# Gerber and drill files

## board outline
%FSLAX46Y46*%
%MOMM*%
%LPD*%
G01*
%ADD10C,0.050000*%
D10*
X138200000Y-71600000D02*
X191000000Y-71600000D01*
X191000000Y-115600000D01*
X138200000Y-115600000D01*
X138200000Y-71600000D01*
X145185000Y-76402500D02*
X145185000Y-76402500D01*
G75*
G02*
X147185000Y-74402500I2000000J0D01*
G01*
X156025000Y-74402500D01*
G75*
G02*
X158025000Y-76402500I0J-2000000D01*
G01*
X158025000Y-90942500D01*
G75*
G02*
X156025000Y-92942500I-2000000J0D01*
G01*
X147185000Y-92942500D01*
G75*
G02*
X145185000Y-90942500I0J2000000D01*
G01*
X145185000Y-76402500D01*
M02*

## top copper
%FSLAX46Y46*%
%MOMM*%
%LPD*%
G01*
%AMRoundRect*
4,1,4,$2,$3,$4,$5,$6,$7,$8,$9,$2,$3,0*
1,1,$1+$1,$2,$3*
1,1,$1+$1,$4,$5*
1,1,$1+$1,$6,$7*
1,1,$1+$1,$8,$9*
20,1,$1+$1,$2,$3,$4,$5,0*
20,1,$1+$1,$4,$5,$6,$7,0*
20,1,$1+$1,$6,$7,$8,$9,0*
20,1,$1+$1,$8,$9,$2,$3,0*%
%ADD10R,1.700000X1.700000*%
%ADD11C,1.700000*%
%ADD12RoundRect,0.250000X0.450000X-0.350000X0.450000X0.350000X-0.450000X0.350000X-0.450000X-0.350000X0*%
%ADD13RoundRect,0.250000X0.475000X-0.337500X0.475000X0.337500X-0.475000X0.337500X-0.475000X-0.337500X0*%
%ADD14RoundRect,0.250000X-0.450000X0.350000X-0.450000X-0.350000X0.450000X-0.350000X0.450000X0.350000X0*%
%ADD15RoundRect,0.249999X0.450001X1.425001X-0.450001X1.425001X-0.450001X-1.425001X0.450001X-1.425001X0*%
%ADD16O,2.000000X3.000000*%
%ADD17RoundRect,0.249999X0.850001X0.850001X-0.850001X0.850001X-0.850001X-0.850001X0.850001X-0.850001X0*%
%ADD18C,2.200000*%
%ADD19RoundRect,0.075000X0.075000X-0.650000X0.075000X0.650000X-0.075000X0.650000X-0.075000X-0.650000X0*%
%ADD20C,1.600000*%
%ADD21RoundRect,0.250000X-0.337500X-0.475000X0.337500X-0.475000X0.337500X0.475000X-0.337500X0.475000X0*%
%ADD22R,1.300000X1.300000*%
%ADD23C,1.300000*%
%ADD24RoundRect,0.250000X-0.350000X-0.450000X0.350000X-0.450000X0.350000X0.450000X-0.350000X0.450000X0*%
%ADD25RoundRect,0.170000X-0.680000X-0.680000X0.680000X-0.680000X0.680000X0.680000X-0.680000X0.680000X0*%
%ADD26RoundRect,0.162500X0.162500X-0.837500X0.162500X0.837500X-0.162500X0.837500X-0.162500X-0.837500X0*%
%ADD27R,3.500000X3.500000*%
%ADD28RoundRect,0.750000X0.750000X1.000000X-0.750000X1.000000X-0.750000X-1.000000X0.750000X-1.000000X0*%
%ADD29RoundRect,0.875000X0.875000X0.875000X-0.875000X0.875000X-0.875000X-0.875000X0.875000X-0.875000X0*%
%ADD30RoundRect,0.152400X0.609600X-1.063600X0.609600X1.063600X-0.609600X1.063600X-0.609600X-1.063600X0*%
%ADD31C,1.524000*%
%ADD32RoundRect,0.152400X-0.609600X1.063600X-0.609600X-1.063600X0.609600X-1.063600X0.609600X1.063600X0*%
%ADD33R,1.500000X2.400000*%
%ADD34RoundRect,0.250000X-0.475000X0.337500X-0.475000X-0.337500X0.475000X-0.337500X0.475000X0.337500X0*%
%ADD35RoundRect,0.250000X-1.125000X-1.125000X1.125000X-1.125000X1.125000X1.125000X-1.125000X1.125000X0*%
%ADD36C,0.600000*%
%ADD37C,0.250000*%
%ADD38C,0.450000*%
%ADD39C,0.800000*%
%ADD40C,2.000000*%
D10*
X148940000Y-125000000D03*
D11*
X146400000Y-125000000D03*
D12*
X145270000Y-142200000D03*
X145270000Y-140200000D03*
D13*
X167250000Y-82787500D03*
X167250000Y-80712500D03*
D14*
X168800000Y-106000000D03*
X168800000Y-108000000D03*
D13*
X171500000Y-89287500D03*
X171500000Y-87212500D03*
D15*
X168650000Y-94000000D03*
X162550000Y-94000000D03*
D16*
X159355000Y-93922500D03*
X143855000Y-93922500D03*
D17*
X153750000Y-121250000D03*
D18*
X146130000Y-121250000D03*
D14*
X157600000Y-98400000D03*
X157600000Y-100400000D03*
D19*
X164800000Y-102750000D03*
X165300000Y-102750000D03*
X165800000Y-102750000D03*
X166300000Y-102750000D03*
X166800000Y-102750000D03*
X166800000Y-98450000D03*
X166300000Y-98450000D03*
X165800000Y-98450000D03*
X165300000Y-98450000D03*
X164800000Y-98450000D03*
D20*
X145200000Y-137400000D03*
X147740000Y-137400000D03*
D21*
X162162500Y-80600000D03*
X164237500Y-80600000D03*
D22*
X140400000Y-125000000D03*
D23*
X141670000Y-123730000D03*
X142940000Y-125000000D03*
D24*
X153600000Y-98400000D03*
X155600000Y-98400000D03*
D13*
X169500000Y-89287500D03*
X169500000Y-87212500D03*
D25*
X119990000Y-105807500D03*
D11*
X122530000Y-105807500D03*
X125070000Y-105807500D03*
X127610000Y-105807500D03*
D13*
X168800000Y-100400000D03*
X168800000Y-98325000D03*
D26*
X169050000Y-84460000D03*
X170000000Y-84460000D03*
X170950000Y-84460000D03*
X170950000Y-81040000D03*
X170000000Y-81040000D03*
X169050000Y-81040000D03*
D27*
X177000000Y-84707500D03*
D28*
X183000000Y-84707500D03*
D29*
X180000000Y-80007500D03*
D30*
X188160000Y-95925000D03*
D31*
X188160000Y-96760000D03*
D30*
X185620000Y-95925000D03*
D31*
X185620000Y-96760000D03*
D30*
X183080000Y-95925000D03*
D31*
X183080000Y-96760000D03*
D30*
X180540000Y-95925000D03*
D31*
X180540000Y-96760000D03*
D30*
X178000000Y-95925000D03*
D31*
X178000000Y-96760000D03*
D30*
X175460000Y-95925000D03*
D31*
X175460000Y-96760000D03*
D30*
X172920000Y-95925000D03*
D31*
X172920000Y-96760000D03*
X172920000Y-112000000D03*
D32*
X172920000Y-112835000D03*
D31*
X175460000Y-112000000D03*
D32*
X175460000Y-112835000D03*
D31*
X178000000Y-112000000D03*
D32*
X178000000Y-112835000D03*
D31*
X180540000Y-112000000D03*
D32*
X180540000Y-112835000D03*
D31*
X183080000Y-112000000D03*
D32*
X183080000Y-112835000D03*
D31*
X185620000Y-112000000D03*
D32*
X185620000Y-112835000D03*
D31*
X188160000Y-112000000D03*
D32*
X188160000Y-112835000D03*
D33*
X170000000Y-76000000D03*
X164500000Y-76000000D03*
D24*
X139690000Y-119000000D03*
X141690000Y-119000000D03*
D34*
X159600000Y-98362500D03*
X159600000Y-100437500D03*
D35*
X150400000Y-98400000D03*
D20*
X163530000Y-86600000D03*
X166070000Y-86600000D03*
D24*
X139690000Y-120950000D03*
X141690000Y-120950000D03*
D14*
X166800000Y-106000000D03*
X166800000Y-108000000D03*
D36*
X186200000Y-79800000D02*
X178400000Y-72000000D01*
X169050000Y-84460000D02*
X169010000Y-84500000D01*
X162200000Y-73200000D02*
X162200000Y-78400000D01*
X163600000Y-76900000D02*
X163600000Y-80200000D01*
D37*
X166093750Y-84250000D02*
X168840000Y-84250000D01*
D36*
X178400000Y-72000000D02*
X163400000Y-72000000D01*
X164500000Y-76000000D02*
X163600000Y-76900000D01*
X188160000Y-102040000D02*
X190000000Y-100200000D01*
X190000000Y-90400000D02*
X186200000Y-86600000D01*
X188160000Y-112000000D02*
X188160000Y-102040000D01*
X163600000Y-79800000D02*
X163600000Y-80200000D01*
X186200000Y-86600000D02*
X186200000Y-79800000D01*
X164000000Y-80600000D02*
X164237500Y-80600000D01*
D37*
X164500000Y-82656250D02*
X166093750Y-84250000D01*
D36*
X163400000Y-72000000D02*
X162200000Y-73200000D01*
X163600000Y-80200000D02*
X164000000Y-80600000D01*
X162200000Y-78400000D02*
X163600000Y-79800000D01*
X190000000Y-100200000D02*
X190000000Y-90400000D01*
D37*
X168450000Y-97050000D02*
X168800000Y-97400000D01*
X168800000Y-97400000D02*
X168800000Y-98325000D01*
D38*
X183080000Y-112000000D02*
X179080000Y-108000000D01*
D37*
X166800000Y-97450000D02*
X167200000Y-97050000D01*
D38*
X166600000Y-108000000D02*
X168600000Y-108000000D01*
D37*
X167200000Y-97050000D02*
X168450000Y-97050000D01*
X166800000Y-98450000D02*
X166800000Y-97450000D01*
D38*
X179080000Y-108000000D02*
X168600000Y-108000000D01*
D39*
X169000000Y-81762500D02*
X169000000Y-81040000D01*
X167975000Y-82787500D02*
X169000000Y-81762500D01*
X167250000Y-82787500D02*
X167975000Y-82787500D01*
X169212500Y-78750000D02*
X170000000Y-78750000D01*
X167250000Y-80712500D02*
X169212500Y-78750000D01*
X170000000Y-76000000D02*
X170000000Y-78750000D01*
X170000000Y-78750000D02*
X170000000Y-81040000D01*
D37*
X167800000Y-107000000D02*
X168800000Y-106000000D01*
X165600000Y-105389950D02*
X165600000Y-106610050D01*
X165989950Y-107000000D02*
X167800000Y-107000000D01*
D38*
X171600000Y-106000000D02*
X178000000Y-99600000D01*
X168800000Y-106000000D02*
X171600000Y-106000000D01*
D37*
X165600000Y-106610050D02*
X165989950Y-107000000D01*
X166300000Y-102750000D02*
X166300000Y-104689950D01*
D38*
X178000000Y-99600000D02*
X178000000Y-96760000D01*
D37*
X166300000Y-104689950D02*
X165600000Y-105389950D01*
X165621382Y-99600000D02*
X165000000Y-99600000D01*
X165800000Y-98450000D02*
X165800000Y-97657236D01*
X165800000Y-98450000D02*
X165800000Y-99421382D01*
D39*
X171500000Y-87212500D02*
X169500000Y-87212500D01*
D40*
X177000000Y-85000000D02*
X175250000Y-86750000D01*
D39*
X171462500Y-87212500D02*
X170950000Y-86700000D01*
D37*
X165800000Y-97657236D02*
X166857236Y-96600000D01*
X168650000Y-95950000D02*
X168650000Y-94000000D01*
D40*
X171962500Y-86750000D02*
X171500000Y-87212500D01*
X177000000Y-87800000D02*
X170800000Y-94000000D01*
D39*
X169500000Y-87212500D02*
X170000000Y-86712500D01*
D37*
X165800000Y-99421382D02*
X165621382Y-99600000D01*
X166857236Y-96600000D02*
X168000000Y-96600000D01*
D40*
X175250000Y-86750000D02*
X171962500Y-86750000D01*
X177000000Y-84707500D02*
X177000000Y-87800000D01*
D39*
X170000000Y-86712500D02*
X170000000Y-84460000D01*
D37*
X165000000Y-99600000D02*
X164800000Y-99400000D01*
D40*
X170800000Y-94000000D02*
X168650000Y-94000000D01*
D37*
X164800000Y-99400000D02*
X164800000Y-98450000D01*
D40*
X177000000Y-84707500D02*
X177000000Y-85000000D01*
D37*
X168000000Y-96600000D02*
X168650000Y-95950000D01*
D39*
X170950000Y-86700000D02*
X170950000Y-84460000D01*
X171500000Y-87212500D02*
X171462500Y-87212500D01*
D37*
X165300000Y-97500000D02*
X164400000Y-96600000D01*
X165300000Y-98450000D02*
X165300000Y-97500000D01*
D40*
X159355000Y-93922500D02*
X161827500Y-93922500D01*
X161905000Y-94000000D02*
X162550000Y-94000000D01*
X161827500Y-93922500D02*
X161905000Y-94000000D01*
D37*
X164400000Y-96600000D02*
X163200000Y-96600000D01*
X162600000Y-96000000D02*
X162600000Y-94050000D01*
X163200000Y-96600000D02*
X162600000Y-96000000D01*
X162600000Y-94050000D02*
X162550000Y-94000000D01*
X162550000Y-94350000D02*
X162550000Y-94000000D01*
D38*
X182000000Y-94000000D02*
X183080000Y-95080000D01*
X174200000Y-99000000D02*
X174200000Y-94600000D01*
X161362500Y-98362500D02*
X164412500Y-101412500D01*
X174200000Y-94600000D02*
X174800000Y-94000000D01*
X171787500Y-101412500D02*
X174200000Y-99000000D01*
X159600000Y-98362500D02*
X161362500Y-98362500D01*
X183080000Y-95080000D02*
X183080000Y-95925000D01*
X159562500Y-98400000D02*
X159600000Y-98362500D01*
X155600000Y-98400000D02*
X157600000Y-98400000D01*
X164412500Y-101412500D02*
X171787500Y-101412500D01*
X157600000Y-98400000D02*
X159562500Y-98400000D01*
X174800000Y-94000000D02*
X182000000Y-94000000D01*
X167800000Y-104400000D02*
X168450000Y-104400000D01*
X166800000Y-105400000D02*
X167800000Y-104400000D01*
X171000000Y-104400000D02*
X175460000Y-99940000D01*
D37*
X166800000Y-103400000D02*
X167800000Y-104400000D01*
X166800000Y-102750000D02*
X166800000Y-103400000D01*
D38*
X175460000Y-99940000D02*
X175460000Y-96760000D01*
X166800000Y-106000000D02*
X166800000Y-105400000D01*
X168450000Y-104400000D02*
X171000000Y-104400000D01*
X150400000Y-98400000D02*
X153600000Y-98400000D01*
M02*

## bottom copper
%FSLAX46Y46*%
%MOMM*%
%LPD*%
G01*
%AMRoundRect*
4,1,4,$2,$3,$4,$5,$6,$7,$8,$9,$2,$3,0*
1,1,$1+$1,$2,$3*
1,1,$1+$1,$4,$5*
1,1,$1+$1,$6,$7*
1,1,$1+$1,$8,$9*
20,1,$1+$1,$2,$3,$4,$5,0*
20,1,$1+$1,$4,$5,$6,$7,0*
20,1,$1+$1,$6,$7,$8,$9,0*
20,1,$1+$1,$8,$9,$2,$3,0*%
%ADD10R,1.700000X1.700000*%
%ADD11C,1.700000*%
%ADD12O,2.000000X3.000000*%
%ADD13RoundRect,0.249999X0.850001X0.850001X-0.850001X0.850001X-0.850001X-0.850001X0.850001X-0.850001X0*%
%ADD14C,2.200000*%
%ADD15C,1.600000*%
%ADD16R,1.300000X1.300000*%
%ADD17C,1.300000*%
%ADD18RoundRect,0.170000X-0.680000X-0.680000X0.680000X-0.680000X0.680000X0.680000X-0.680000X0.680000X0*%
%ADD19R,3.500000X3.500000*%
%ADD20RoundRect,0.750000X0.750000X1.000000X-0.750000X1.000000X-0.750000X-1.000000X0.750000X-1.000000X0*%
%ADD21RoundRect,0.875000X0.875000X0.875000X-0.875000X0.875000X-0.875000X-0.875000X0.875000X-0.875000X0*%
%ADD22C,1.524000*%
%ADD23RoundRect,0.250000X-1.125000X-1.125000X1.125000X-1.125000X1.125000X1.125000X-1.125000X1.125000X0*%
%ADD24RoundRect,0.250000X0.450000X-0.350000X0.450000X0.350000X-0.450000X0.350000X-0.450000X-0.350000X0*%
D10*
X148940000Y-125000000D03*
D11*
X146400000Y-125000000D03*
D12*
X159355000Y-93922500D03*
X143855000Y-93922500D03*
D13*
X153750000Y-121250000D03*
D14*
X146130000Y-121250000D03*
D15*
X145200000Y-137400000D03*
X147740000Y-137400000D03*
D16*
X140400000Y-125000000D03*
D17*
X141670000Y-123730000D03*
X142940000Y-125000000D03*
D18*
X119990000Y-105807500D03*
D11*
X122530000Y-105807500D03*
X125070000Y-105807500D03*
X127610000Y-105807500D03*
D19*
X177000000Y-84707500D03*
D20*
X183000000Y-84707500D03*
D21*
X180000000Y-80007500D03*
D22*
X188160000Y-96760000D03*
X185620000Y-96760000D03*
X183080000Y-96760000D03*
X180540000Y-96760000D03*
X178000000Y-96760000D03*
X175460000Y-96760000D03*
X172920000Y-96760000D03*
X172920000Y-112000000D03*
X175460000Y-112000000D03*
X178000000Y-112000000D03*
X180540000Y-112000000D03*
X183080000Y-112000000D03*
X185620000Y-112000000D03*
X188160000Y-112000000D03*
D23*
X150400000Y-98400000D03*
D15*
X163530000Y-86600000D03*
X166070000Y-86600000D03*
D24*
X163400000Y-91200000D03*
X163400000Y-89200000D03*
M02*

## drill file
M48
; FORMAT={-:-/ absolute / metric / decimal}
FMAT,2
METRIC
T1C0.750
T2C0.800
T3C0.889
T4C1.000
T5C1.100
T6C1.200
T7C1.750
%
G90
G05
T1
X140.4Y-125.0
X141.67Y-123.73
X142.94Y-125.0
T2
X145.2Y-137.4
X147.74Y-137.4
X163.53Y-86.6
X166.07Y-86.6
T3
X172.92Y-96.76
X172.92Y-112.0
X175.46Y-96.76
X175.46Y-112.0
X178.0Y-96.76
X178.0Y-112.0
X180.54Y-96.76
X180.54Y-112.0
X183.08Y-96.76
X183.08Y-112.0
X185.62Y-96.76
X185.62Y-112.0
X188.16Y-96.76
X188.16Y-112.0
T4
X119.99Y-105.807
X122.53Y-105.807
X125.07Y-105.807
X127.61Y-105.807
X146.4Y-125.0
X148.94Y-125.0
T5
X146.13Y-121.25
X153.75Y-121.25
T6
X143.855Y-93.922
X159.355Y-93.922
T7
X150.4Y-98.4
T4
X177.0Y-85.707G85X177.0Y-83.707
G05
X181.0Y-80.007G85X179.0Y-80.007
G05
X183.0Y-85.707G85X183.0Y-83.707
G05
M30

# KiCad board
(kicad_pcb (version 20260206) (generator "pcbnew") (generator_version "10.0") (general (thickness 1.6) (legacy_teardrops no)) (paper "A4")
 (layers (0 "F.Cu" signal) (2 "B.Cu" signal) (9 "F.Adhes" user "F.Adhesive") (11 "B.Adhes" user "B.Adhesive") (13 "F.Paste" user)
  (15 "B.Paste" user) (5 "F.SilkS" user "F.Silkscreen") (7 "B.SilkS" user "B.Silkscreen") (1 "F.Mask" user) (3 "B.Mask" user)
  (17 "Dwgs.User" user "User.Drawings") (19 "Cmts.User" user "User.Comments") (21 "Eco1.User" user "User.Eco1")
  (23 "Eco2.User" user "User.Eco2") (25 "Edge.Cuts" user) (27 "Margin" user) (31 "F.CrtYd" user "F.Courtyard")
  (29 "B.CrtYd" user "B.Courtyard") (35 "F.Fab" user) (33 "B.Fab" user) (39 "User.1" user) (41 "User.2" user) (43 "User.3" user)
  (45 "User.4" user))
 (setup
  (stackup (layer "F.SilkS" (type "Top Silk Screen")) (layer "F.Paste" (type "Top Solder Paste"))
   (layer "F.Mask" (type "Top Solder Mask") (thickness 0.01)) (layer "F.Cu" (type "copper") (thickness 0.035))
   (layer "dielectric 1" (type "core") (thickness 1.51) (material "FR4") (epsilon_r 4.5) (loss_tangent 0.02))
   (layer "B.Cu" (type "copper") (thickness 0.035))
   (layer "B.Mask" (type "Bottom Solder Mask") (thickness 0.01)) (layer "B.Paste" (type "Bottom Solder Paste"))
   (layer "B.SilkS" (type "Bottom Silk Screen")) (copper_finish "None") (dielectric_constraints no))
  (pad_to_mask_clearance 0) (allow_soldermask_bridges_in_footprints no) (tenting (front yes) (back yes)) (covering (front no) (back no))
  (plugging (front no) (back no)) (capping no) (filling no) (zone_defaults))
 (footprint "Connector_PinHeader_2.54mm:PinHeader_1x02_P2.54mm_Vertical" (layer "F.Cu") (at 148.94 125 -90)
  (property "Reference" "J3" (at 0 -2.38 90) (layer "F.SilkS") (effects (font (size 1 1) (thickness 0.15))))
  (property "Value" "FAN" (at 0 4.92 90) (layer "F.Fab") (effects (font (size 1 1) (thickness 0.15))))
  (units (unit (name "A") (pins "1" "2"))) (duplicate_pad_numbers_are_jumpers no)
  (pad "1" thru_hole rect (at 0 0 270) (size 1.7 1.7) (drill 1) (layers "*.Cu" "*.Mask") (remove_unused_layers no) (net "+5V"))
  (pad "2" thru_hole circle (at 0 2.54 270) (size 1.7 1.7) (drill 1) (layers "*.Cu" "*.Mask") (remove_unused_layers no) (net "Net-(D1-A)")))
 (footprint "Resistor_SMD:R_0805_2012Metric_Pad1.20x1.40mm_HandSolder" (layer "F.Cu") (at 145.27 141.2 90)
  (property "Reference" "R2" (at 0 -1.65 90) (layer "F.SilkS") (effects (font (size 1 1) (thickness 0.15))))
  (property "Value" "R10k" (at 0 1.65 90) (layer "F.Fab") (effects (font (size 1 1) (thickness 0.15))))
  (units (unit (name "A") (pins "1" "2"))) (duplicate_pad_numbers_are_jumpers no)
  (pad "1" smd roundrect (at -1 0 90) (size 1.2 1.4) (layers "F.Cu" "F.Mask" "F.Paste") (roundrect_rratio 0.208333) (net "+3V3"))
  (pad "2" smd roundrect (at 1 0 90) (size 1.2 1.4) (layers "F.Cu" "F.Mask" "F.Paste") (roundrect_rratio 0.208333) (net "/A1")))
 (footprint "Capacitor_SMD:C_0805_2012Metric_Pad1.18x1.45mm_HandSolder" (layer "F.Cu") (at 167.25 81.75 90)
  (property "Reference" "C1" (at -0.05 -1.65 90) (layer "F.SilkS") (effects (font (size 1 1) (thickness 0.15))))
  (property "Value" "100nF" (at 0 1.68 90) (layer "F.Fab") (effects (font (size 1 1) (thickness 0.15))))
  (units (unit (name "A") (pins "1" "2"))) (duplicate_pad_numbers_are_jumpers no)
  (pad "1" smd roundrect (at -1.0375 0 90) (size 1.175 1.45) (layers "F.Cu" "F.Mask" "F.Paste") (roundrect_rratio 0.212766)
   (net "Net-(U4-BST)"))
  (pad "2" smd roundrect (at 1.0375 0 90) (size 1.175 1.45) (layers "F.Cu" "F.Mask" "F.Paste") (roundrect_rratio 0.212766)
   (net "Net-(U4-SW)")))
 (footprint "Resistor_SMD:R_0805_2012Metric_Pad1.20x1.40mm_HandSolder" (layer "F.Cu") (at 168.8 107 -90)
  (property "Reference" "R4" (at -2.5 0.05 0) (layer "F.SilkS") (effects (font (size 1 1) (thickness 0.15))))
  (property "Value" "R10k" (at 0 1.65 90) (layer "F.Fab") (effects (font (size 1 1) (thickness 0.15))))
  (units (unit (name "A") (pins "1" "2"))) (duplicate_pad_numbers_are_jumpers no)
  (pad "1" smd roundrect (at -1 0 270) (size 1.2 1.4) (layers "F.Cu" "F.Mask" "F.Paste") (roundrect_rratio 0.208333) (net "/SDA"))
  (pad "2" smd roundrect (at 1 0 270) (size 1.2 1.4) (layers "F.Cu" "F.Mask" "F.Paste") (roundrect_rratio 0.208333) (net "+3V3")))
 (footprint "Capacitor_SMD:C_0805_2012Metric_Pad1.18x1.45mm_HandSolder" (layer "F.Cu") (at 171.5 88.25 90)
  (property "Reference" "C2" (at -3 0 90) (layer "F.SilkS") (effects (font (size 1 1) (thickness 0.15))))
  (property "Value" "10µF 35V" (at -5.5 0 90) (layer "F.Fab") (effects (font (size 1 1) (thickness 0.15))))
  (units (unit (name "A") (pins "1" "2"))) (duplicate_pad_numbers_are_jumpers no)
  (pad "1" smd roundrect (at -1.0375 0 90) (size 1.175 1.45) (layers "F.Cu" "F.Mask" "F.Paste") (roundrect_rratio 0.212766) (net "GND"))
  (pad "2" smd roundrect (at 1.0375 0 90) (size 1.175 1.45) (layers "F.Cu" "F.Mask" "F.Paste") (roundrect_rratio 0.212766) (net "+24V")))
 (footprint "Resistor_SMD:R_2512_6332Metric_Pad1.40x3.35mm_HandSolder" (layer "F.Cu") (at 165.6 94 180)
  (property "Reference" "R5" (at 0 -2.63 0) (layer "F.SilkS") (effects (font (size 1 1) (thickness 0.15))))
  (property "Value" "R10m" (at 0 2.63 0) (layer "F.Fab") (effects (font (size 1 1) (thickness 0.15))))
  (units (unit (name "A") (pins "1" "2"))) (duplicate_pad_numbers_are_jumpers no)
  (pad "1" smd roundrect (at -3.05 0 180) (size 1.4 3.35) (layers "F.Cu" "F.Mask" "F.Paste") (roundrect_rratio 0.178571) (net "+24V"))
  (pad "2" smd roundrect (at 3.05 0 180) (size 1.4 3.35) (layers "F.Cu" "F.Mask" "F.Paste") (roundrect_rratio 0.178571) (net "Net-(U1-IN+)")))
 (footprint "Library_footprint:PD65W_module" (layer "F.Cu") (at 151.605 83.6725 -90)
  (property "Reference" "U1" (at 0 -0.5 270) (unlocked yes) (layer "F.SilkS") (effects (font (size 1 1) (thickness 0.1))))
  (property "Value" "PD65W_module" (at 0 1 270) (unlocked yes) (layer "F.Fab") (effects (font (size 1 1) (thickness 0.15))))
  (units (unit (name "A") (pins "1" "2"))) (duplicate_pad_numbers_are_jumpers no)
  (fp_rect (start -9.27 -6.42) (end 9.27 6.42) (radius 2) (stroke (width 0.05) (type solid)) (fill no) (layer "Edge.Cuts"))
  (pad "1" thru_hole oval (at 10.25 -7.75 270) (size 3 2) (drill 1.2) (layers "*.Cu" "*.Mask") (remove_unused_layers no)
   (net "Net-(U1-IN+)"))
  (pad "2" thru_hole oval (at 10.25 7.75 270) (size 3 2) (drill 1.2) (layers "*.Cu" "*.Mask") (remove_unused_layers no) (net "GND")))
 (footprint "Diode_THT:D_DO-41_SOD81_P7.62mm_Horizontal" (layer "F.Cu") (at 153.75 121.25 180)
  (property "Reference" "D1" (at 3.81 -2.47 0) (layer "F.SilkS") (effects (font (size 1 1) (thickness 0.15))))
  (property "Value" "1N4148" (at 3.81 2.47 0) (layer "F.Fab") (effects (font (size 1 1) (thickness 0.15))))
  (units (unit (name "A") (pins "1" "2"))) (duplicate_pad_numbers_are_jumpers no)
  (pad "1" thru_hole roundrect (at 0 0 180) (size 2.2 2.2) (drill 1.1) (layers "*.Cu" "*.Mask") (remove_unused_layers no)
   (roundrect_rratio 0.113636) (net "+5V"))
  (pad "2" thru_hole circle (at 7.62 0 180) (size 2.2 2.2) (drill 1.1) (layers "*.Cu" "*.Mask") (remove_unused_layers no) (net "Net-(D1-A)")))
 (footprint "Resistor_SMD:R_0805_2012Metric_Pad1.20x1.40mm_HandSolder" (layer "F.Cu") (at 157.6 99.4 -90)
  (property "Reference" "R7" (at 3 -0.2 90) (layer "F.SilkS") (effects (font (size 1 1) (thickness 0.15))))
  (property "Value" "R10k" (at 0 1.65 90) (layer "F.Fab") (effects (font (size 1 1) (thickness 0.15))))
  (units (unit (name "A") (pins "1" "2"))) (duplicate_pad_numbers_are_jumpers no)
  (pad "1" smd roundrect (at -1 0 270) (size 1.2 1.4) (layers "F.Cu" "F.Mask" "F.Paste") (roundrect_rratio 0.208333) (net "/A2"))
  (pad "2" smd roundrect (at 1 0 270) (size 1.2 1.4) (layers "F.Cu" "F.Mask" "F.Paste") (roundrect_rratio 0.208333) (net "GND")))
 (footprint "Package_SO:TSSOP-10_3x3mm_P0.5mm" (layer "F.Cu") (at 165.8 100.6 90)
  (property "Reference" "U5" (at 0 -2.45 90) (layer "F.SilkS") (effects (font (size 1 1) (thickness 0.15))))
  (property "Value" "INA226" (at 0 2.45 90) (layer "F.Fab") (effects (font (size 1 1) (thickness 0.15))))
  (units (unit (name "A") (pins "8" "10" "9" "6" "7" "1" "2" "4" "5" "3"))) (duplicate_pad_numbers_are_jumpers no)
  (pad "1" smd roundrect (at -2.15 -1 90) (size 1.45 0.3) (layers "F.Cu" "F.Mask" "F.Paste") (roundrect_rratio 0.25) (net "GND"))
  (pad "2" smd roundrect (at -2.15 -0.5 90) (size 1.45 0.3) (layers "F.Cu" "F.Mask" "F.Paste") (roundrect_rratio 0.25) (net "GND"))
  (pad "3" smd roundrect (at -2.15 0 90) (size 1.45 0.3) (layers "F.Cu" "F.Mask" "F.Paste") (roundrect_rratio 0.25)
   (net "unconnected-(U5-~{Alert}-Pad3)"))
  (pad "4" smd roundrect (at -2.15 0.5 90) (size 1.45 0.3) (layers "F.Cu" "F.Mask" "F.Paste") (roundrect_rratio 0.25) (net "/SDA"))
  (pad "5" smd roundrect (at -2.15 1 90) (size 1.45 0.3) (layers "F.Cu" "F.Mask" "F.Paste") (roundrect_rratio 0.25) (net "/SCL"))
  (pad "6" smd roundrect (at 2.15 1 90) (size 1.45 0.3) (layers "F.Cu" "F.Mask" "F.Paste") (roundrect_rratio 0.25) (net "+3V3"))
  (pad "7" smd roundrect (at 2.15 0.5 90) (size 1.45 0.3) (layers "F.Cu" "F.Mask" "F.Paste") (roundrect_rratio 0.25) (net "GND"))
  (pad "8" smd roundrect (at 2.15 0 90) (size 1.45 0.3) (layers "F.Cu" "F.Mask" "F.Paste") (roundrect_rratio 0.25) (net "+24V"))
  (pad "9" smd roundrect (at 2.15 -0.5 90) (size 1.45 0.3) (layers "F.Cu" "F.Mask" "F.Paste") (roundrect_rratio 0.25) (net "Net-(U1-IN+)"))
  (pad "10" smd roundrect (at 2.15 -1 90) (size 1.45 0.3) (layers "F.Cu" "F.Mask" "F.Paste") (roundrect_rratio 0.25) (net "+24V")))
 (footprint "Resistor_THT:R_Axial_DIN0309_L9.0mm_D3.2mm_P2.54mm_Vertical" (layer "F.Cu") (at 145.2 137.4)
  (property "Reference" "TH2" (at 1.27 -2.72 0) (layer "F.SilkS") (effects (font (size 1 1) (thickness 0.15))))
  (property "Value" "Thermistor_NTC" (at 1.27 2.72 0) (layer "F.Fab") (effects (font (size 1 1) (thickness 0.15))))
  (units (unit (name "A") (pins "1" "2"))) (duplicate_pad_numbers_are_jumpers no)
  (pad "1" thru_hole circle (at 0 0) (size 1.6 1.6) (drill 0.8) (layers "*.Cu" "*.Mask") (remove_unused_layers no) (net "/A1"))
  (pad "2" thru_hole circle (at 2.54 0) (size 1.6 1.6) (drill 0.8) (layers "*.Cu" "*.Mask") (remove_unused_layers no) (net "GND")))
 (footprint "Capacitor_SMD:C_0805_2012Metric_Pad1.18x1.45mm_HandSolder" (layer "F.Cu") (at 163.2 80.6)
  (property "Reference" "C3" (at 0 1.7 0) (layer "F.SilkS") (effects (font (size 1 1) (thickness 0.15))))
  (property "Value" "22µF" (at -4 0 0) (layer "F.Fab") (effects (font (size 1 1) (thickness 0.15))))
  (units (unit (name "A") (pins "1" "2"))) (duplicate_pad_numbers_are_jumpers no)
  (pad "1" smd roundrect (at -1.0375 0) (size 1.175 1.45) (layers "F.Cu" "F.Mask" "F.Paste") (roundrect_rratio 0.212766) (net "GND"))
  (pad "2" smd roundrect (at 1.0375 0) (size 1.175 1.45) (layers "F.Cu" "F.Mask" "F.Paste") (roundrect_rratio 0.212766) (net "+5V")))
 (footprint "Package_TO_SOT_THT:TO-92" (layer "F.Cu") (at 140.4 125)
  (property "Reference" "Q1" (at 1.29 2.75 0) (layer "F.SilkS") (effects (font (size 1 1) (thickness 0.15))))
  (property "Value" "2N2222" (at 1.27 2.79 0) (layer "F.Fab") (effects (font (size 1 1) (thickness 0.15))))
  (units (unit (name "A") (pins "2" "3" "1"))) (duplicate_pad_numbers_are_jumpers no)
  (pad "1" thru_hole rect (at 0 0) (size 1.3 1.3) (drill 0.75) (layers "*.Cu" "*.Mask") (remove_unused_layers no) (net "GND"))
  (pad "2" thru_hole circle (at 1.27 -1.27) (size 1.3 1.3) (drill 0.75) (layers "*.Cu" "*.Mask") (remove_unused_layers no)
   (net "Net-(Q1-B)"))
  (pad "3" thru_hole circle (at 2.54 0) (size 1.3 1.3) (drill 0.75) (layers "*.Cu" "*.Mask") (remove_unused_layers no) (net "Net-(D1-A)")))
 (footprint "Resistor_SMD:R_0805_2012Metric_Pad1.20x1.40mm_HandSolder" (layer "F.Cu") (at 154.6 98.4)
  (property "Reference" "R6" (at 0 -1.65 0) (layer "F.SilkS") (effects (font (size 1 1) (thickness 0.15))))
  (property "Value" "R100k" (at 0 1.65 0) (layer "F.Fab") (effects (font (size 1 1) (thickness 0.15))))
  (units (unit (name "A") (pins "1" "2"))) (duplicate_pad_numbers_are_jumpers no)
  (pad "1" smd roundrect (at -1 0) (size 1.2 1.4) (layers "F.Cu" "F.Mask" "F.Paste") (roundrect_rratio 0.208333) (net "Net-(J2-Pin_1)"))
  (pad "2" smd roundrect (at 1 0) (size 1.2 1.4) (layers "F.Cu" "F.Mask" "F.Paste") (roundrect_rratio 0.208333) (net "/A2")))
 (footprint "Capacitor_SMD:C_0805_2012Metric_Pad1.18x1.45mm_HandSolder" (layer "F.Cu") (at 169.5 88.25 90)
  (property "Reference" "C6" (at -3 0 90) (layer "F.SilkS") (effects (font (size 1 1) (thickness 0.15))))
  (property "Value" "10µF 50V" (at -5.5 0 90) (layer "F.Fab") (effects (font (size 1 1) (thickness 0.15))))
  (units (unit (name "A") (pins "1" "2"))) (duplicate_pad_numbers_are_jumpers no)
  (pad "1" smd roundrect (at -1.0375 0 90) (size 1.175 1.45) (layers "F.Cu" "F.Mask" "F.Paste") (roundrect_rratio 0.212766) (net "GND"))
  (pad "2" smd roundrect (at 1.0375 0 90) (size 1.175 1.45) (layers "F.Cu" "F.Mask" "F.Paste") (roundrect_rratio 0.212766) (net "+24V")))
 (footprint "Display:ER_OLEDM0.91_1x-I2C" (layer "F.Cu") (at 119.99 105.8075)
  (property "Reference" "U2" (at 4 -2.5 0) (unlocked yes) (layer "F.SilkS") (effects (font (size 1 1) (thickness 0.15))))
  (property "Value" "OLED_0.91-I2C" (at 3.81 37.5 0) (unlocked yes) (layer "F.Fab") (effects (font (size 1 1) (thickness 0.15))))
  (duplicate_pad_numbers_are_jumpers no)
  (pad "1" thru_hole roundrect (at 0 0) (size 1.7 1.7) (drill 1) (layers "*.Cu" "*.Mask") (remove_unused_layers no) (roundrect_rratio 0.1)
   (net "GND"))
  (pad "2" thru_hole circle (at 2.54 0) (size 1.7 1.7) (drill 1) (layers "*.Cu" "*.Mask") (remove_unused_layers no) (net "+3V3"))
  (pad "3" thru_hole circle (at 5.08 0) (size 1.7 1.7) (drill 1) (layers "*.Cu" "*.Mask") (remove_unused_layers no) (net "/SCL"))
  (pad "4" thru_hole circle (at 7.62 0) (size 1.7 1.7) (drill 1) (layers "*.Cu" "*.Mask") (remove_unused_layers no) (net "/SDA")))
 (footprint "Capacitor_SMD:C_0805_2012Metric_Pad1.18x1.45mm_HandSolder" (layer "F.Cu") (at 168.8 99.3625 90)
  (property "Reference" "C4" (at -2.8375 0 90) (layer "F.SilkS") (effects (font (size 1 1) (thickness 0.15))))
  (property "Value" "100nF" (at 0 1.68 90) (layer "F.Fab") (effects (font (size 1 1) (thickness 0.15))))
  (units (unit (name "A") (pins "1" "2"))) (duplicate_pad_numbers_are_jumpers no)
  (pad "1" smd roundrect (at -1.0375 0 90) (size 1.175 1.45) (layers "F.Cu" "F.Mask" "F.Paste") (roundrect_rratio 0.212766) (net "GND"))
  (pad "2" smd roundrect (at 1.0375 0 90) (size 1.175 1.45) (layers "F.Cu" "F.Mask" "F.Paste") (roundrect_rratio 0.212766) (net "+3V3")))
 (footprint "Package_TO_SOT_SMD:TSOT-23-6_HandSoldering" (layer "F.Cu") (at 170 82.75 90)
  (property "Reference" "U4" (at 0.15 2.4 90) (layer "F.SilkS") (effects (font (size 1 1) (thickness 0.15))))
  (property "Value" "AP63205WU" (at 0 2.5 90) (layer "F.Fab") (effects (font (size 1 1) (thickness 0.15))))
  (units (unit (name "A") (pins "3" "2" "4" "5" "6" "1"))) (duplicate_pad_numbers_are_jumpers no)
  (pad "1" smd roundrect (at -1.71 -0.95 90) (size 2 0.65) (layers "F.Cu" "F.Mask" "F.Paste") (roundrect_rratio 0.25) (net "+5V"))
  (pad "2" smd roundrect (at -1.71 0 90) (size 2 0.65) (layers "F.Cu" "F.Mask" "F.Paste") (roundrect_rratio 0.25) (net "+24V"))
  (pad "3" smd roundrect (at -1.71 0.95 90) (size 2 0.65) (layers "F.Cu" "F.Mask" "F.Paste") (roundrect_rratio 0.25) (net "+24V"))
  (pad "4" smd roundrect (at 1.71 0.95 90) (size 2 0.65) (layers "F.Cu" "F.Mask" "F.Paste") (roundrect_rratio 0.25) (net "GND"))
  (pad "5" smd roundrect (at 1.71 0 90) (size 2 0.65) (layers "F.Cu" "F.Mask" "F.Paste") (roundrect_rratio 0.25) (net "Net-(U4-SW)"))
  (pad "6" smd roundrect (at 1.71 -0.95 90) (size 2 0.65) (layers "F.Cu" "F.Mask" "F.Paste") (roundrect_rratio 0.25) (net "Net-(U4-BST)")))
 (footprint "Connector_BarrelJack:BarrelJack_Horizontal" (layer "F.Cu") (at 177 84.7075 180)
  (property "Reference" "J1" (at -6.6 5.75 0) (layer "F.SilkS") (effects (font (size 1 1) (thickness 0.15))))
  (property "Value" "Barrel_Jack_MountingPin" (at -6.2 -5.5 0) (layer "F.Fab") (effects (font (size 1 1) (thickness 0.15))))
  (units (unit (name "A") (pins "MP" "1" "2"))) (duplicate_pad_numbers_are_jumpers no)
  (pad "1" thru_hole rect (at 0 0 180) (size 3.5 3.5) (drill oval 1 3) (layers "*.Cu" "*.Mask") (remove_unused_layers no) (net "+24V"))
  (pad "2" thru_hole roundrect (at -6 0 180) (size 3 3.5) (drill oval 1 3) (layers "*.Cu" "*.Mask") (remove_unused_layers no)
   (roundrect_rratio 0.25) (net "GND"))
  (pad "3" thru_hole roundrect (at -3 4.7 180) (size 3.5 3.5) (drill oval 3 1) (layers "*.Cu" "*.Mask") (remove_unused_layers no)
   (roundrect_rratio 0.25)))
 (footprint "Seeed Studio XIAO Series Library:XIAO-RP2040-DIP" (layer "F.Cu") (at 180.54 104.38 -90)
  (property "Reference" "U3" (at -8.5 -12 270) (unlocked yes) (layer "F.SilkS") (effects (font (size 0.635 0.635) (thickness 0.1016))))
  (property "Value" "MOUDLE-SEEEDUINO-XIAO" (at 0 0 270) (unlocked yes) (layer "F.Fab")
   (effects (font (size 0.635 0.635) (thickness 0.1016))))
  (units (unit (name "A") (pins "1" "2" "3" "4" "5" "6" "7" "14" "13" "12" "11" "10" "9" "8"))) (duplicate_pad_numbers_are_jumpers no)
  (pad "1" smd roundrect (at -8.455 -7.62 90) (size 2.432 1.524) (layers "F.Cu" "F.Mask") (roundrect_rratio 0.1) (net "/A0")
   (thermal_bridge_angle 45))
  (pad "1" thru_hole circle (at -7.62 -7.62 90) (size 1.524 1.524) (drill 0.889) (layers "*.Cu" "*.Mask") (remove_unused_layers no)
   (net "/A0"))
  (pad "2" smd roundrect (at -8.455 -5.08 90) (size 2.432 1.524) (layers "F.Cu" "F.Mask") (roundrect_rratio 0.1) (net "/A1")
   (thermal_bridge_angle 45))
  (pad "2" thru_hole circle (at -7.62 -5.08 90) (size 1.524 1.524) (drill 0.889) (layers "*.Cu" "*.Mask") (remove_unused_layers no)
   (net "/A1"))
  (pad "3" smd roundrect (at -8.455 -2.54 90) (size 2.432 1.524) (layers "F.Cu" "F.Mask") (roundrect_rratio 0.1) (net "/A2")
   (thermal_bridge_angle 45))
  (pad "3" thru_hole circle (at -7.62 -2.54 90) (size 1.524 1.524) (drill 0.889) (layers "*.Cu" "*.Mask") (remove_unused_layers no)
   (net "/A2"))
  (pad "4" smd roundrect (at -8.455 0 90) (size 2.432 1.524) (layers "F.Cu" "F.Mask") (roundrect_rratio 0.1) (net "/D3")
   (thermal_bridge_angle 45))
  (pad "4" thru_hole circle (at -7.62 0 90) (size 1.524 1.524) (drill 0.889) (layers "*.Cu" "*.Mask") (remove_unused_layers no) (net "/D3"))
  (pad "5" smd roundrect (at -8.455 2.54 90) (size 2.432 1.524) (layers "F.Cu" "F.Mask") (roundrect_rratio 0.1) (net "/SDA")
   (thermal_bridge_angle 45))
  (pad "5" thru_hole circle (at -7.62 2.54 90) (size 1.524 1.524) (drill 0.889) (layers "*.Cu" "*.Mask") (remove_unused_layers no)
   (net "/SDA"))
  (pad "6" smd roundrect (at -8.455 5.08 90) (size 2.432 1.524) (layers "F.Cu" "F.Mask") (roundrect_rratio 0.1) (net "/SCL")
   (thermal_bridge_angle 45))
  (pad "6" thru_hole circle (at -7.62 5.08 90) (size 1.524 1.524) (drill 0.889) (layers "*.Cu" "*.Mask") (remove_unused_layers no)
   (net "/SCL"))
  (pad "7" smd roundrect (at -8.455 7.62 90) (size 2.432 1.524) (layers "F.Cu" "F.Mask") (roundrect_rratio 0.1)
   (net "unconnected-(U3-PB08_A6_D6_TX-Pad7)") (thermal_bridge_angle 45))
  (pad "7" thru_hole circle (at -7.62 7.62 90) (size 1.524 1.524) (drill 0.889) (layers "*.Cu" "*.Mask") (remove_unused_layers no)
   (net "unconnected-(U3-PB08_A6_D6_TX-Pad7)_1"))
  (pad "8" thru_hole circle (at 7.62 7.62 270) (size 1.524 1.524) (drill 0.889) (layers "*.Cu" "*.Mask") (remove_unused_layers no)
   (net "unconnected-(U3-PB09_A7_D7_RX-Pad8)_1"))
  (pad "8" smd roundrect (at 8.455 7.62 270) (size 2.432 1.524) (layers "F.Cu" "F.Mask") (roundrect_rratio 0.1)
   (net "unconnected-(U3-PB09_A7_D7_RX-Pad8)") (thermal_bridge_angle 45))
  (pad "9" thru_hole circle (at 7.62 5.08 270) (size 1.524 1.524) (drill 0.889) (layers "*.Cu" "*.Mask") (remove_unused_layers no)
   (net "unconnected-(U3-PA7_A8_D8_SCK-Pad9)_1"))
  (pad "9" smd roundrect (at 8.455 5.08 270) (size 2.432 1.524) (layers "F.Cu" "F.Mask") (roundrect_rratio 0.1)
   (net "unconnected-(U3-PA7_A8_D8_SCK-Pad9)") (thermal_bridge_angle 45))
  (pad "10" thru_hole circle (at 7.62 2.54 270) (size 1.524 1.524) (drill 0.889) (layers "*.Cu" "*.Mask") (remove_unused_layers no)
   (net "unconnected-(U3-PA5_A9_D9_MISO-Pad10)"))
  (pad "10" smd roundrect (at 8.455 2.54 270) (size 2.432 1.524) (layers "F.Cu" "F.Mask") (roundrect_rratio 0.1)
   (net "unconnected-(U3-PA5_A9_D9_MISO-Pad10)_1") (thermal_bridge_angle 45))
  (pad "11" thru_hole circle (at 7.62 0 270) (size 1.524 1.524) (drill 0.889) (layers "*.Cu" "*.Mask") (remove_unused_layers no)
   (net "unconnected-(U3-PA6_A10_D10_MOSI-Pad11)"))
  (pad "11" smd roundrect (at 8.455 0 270) (size 2.432 1.524) (layers "F.Cu" "F.Mask") (roundrect_rratio 0.1)
   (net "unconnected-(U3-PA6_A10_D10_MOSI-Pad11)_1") (thermal_bridge_angle 45))
  (pad "12" thru_hole circle (at 7.62 -2.54 270) (size 1.524 1.524) (drill 0.889) (layers "*.Cu" "*.Mask") (remove_unused_layers no)
   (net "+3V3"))
  (pad "12" smd roundrect (at 8.455 -2.54 270) (size 2.432 1.524) (layers "F.Cu" "F.Mask") (roundrect_rratio 0.1) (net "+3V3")
   (thermal_bridge_angle 45))
  (pad "13" thru_hole circle (at 7.62 -5.08 270) (size 1.524 1.524) (drill 0.889) (layers "*.Cu" "*.Mask") (remove_unused_layers no)
   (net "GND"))
  (pad "13" smd roundrect (at 8.455 -5.08 270) (size 2.432 1.524) (layers "F.Cu" "F.Mask") (roundrect_rratio 0.1) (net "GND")
   (thermal_bridge_angle 45))
  (pad "14" thru_hole circle (at 7.62 -7.62 270) (size 1.524 1.524) (drill 0.889) (layers "*.Cu" "*.Mask") (remove_unused_layers no)
   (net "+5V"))
  (pad "14" smd roundrect (at 8.455 -7.62 270) (size 2.432 1.524) (layers "F.Cu" "F.Mask") (roundrect_rratio 0.1) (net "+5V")
   (thermal_bridge_angle 45)))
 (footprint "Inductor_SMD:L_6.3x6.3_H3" (layer "F.Cu") (at 167.25 76 180)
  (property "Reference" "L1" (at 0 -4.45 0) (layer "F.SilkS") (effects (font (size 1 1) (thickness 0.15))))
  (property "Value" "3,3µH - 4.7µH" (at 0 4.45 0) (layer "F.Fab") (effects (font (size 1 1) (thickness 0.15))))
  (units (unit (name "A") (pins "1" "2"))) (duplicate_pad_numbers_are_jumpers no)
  (pad "1" smd rect (at -2.75 0 180) (size 1.5 2.4) (layers "F.Cu" "F.Mask" "F.Paste") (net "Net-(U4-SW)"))
  (pad "2" smd rect (at 2.75 0 180) (size 1.5 2.4) (layers "F.Cu" "F.Mask" "F.Paste") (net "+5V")))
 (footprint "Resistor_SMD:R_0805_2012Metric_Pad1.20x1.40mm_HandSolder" (layer "F.Cu") (at 140.69 119)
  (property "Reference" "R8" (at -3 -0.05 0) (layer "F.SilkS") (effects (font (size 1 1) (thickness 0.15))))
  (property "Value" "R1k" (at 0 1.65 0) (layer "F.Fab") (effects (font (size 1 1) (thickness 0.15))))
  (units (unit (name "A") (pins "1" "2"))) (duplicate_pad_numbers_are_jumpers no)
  (pad "1" smd roundrect (at -1 0) (size 1.2 1.4) (layers "F.Cu" "F.Mask" "F.Paste") (roundrect_rratio 0.208333) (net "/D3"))
  (pad "2" smd roundrect (at 1 0) (size 1.2 1.4) (layers "F.Cu" "F.Mask" "F.Paste") (roundrect_rratio 0.208333) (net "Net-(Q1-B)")))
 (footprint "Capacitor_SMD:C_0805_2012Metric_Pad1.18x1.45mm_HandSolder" (layer "F.Cu") (at 159.6 99.4 -90)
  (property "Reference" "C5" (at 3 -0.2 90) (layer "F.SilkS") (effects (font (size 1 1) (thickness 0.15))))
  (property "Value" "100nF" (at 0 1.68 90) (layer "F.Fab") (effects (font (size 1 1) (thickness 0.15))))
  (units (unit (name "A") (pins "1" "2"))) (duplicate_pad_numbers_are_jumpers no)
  (pad "1" smd roundrect (at -1.0375 0 270) (size 1.175 1.45) (layers "F.Cu" "F.Mask" "F.Paste") (roundrect_rratio 0.212766) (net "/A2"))
  (pad "2" smd roundrect (at 1.0375 0 270) (size 1.175 1.45) (layers "F.Cu" "F.Mask" "F.Paste") (roundrect_rratio 0.212766) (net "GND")))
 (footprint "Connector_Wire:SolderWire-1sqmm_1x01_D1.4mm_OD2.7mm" (layer "F.Cu") (at 150.4 98.4)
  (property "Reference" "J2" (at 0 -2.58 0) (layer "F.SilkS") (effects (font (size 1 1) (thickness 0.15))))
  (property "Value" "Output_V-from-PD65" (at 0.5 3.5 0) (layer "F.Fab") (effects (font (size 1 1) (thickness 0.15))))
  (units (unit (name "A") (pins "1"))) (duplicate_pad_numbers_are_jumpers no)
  (pad "1" thru_hole roundrect (at 0 0) (size 2.75 2.75) (drill 1.75) (layers "*.Cu" "*.Mask") (remove_unused_layers no)
   (roundrect_rratio 0.090909) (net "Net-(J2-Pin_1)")))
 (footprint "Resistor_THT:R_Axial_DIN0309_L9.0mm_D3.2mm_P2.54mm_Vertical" (layer "F.Cu") (at 163.53 86.6)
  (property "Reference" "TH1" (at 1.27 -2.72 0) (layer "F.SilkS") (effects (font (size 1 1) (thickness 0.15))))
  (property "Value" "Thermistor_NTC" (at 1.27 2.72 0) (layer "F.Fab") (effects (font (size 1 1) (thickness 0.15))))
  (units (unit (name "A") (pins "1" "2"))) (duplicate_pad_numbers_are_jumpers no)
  (pad "1" thru_hole circle (at 0 0) (size 1.6 1.6) (drill 0.8) (layers "*.Cu" "*.Mask") (remove_unused_layers no) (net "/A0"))
  (pad "2" thru_hole circle (at 2.54 0) (size 1.6 1.6) (drill 0.8) (layers "*.Cu" "*.Mask") (remove_unused_layers no) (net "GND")))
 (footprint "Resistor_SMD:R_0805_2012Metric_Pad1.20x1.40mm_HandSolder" (layer "F.Cu") (at 140.69 120.95)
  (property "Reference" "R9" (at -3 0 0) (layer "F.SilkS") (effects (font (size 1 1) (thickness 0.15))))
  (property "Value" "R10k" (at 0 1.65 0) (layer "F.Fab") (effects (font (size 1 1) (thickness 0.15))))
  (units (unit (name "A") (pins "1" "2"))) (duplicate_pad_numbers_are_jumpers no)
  (pad "1" smd roundrect (at -1 0) (size 1.2 1.4) (layers "F.Cu" "F.Mask" "F.Paste") (roundrect_rratio 0.208333) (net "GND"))
  (pad "2" smd roundrect (at 1 0) (size 1.2 1.4) (layers "F.Cu" "F.Mask" "F.Paste") (roundrect_rratio 0.208333) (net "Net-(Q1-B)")))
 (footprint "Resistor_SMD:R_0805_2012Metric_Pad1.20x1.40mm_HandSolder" (layer "F.Cu") (at 166.8 107 -90)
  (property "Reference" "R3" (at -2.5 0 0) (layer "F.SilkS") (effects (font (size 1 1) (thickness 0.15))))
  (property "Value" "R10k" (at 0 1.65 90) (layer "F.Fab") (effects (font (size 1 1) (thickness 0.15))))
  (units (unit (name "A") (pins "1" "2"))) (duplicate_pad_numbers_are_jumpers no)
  (pad "1" smd roundrect (at -1 0 270) (size 1.2 1.4) (layers "F.Cu" "F.Mask" "F.Paste") (roundrect_rratio 0.208333) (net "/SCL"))
  (pad "2" smd roundrect (at 1 0 270) (size 1.2 1.4) (layers "F.Cu" "F.Mask" "F.Paste") (roundrect_rratio 0.208333) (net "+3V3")))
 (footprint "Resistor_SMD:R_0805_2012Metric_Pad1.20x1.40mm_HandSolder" (layer "B.Cu") (at 163.4 90.2 90)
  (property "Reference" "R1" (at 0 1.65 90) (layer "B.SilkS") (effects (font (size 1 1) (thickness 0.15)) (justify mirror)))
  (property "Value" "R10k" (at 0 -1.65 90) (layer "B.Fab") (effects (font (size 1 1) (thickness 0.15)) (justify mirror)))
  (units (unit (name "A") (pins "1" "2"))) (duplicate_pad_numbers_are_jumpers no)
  (pad "1" smd roundrect (at -1 0 90) (size 1.2 1.4) (layers "B.Cu" "B.Mask" "B.Paste") (roundrect_rratio 0.208333) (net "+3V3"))
  (pad "2" smd roundrect (at 1 0 90) (size 1.2 1.4) (layers "B.Cu" "B.Mask" "B.Paste") (roundrect_rratio 0.208333) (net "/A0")))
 (gr_rect (start 191 115.6) (end 138.2 71.6) (stroke (width 0.05) (type solid)) (fill no) (layer "Edge.Cuts"))
 (segment (start 186.2 79.8) (end 178.4 72) (width 0.6) (layer "F.Cu") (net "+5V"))
 (segment (start 169.05 84.46) (end 169.01 84.5) (width 0.6) (layer "F.Cu") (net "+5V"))
 (segment (start 162.2 73.2) (end 162.2 78.4) (width 0.6) (layer "F.Cu") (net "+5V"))
 (segment (start 163.6 76.9) (end 163.6 80.2) (width 0.6) (layer "F.Cu") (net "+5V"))
 (segment (start 166.09375 84.25) (end 168.84 84.25) (width 0.25) (layer "F.Cu") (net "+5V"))
 (segment (start 178.4 72) (end 163.4 72) (width 0.6) (layer "F.Cu") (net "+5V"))
 (segment (start 164.5 76) (end 163.6 76.9) (width 0.6) (layer "F.Cu") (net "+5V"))
 (segment (start 188.16 102.04) (end 190 100.2) (width 0.6) (layer "F.Cu") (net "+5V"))
 (segment (start 190 90.4) (end 186.2 86.6) (width 0.6) (layer "F.Cu") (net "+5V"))
 (segment (start 188.16 112) (end 188.16 102.04) (width 0.6) (layer "F.Cu") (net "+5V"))
 (segment (start 163.6 79.8) (end 163.6 80.2) (width 0.6) (layer "F.Cu") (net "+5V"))
 (segment (start 186.2 86.6) (end 186.2 79.8) (width 0.6) (layer "F.Cu") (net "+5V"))
 (segment (start 164 80.6) (end 164.2375 80.6) (width 0.6) (layer "F.Cu") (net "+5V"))
 (segment (start 164.5 82.65625) (end 166.09375 84.25) (width 0.25) (layer "F.Cu") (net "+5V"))
 (segment (start 163.4 72) (end 162.2 73.2) (width 0.6) (layer "F.Cu") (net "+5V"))
 (segment (start 163.6 80.2) (end 164 80.6) (width 0.6) (layer "F.Cu") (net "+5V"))
 (segment (start 162.2 78.4) (end 163.6 79.8) (width 0.6) (layer "F.Cu") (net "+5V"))
 (segment (start 190 100.2) (end 190 90.4) (width 0.6) (layer "F.Cu") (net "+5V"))
 (segment (start 168.45 97.05) (end 168.8 97.4) (width 0.25) (layer "F.Cu") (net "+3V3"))
 (segment (start 168.8 97.4) (end 168.8 98.325) (width 0.25) (layer "F.Cu") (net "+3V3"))
 (segment (start 183.08 112) (end 179.08 108) (width 0.45) (layer "F.Cu") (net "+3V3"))
 (segment (start 166.8 97.45) (end 167.2 97.05) (width 0.25) (layer "F.Cu") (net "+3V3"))
 (segment (start 166.6 108) (end 168.6 108) (width 0.45) (layer "F.Cu") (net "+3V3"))
 (segment (start 167.2 97.05) (end 168.45 97.05) (width 0.25) (layer "F.Cu") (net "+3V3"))
 (segment (start 166.8 98.45) (end 166.8 97.45) (width 0.25) (layer "F.Cu") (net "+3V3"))
 (segment (start 179.08 108) (end 168.6 108) (width 0.45) (layer "F.Cu") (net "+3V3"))
 (segment (start 169 81.7625) (end 169 81.04) (width 0.8) (layer "F.Cu") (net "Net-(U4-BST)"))
 (segment (start 167.975 82.7875) (end 169 81.7625) (width 0.8) (layer "F.Cu") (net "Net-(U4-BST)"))
 (segment (start 167.25 82.7875) (end 167.975 82.7875) (width 0.8) (layer "F.Cu") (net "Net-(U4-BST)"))
 (segment (start 169.2125 78.75) (end 170 78.75) (width 0.8) (layer "F.Cu") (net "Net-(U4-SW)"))
 (segment (start 167.25 80.7125) (end 169.2125 78.75) (width 0.8) (layer "F.Cu") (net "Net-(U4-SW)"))
 (segment (start 170 76) (end 170 78.75) (width 0.8) (layer "F.Cu") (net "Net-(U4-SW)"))
 (segment (start 170 78.75) (end 170 81.04) (width 0.8) (layer "F.Cu") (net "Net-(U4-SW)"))
 (segment (start 167.8 107) (end 168.8 106) (width 0.25) (layer "F.Cu") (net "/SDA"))
 (segment (start 165.6 105.38995) (end 165.6 106.61005) (width 0.25) (layer "F.Cu") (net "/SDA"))
 (segment (start 165.98995 107) (end 167.8 107) (width 0.25) (layer "F.Cu") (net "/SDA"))
 (segment (start 171.6 106) (end 178 99.6) (width 0.45) (layer "F.Cu") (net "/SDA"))
 (segment (start 168.8 106) (end 171.6 106) (width 0.45) (layer "F.Cu") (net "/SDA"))
 (segment (start 165.6 106.61005) (end 165.98995 107) (width 0.25) (layer "F.Cu") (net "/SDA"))
 (segment (start 166.3 102.75) (end 166.3 104.68995) (width 0.25) (layer "F.Cu") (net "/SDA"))
 (segment (start 178 99.6) (end 178 96.76) (width 0.45) (layer "F.Cu") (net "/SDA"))
 (segment (start 166.3 104.68995) (end 165.6 105.38995) (width 0.25) (layer "F.Cu") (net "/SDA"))
 (segment (start 165.621382 99.6) (end 165 99.6) (width 0.25) (layer "F.Cu") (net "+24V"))
 (segment (start 165.8 98.45) (end 165.8 97.657236) (width 0.25) (layer "F.Cu") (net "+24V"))
 (segment (start 165.8 98.45) (end 165.8 99.421382) (width 0.25) (layer "F.Cu") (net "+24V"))
 (segment (start 171.5 87.2125) (end 169.5 87.2125) (width 0.8) (layer "F.Cu") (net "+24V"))
 (segment (start 177 85) (end 175.25 86.75) (width 2) (layer "F.Cu") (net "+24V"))
 (segment (start 171.4625 87.2125) (end 170.95 86.7) (width 0.8) (layer "F.Cu") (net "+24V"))
 (segment (start 165.8 97.657236) (end 166.857236 96.6) (width 0.25) (layer "F.Cu") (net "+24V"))
 (segment (start 168.65 95.95) (end 168.65 94) (width 0.25) (layer "F.Cu") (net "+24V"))
 (segment (start 171.9625 86.75) (end 171.5 87.2125) (width 2) (layer "F.Cu") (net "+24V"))
 (segment (start 177 87.8) (end 170.8 94) (width 2) (layer "F.Cu") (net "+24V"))
 (segment (start 169.5 87.2125) (end 170 86.7125) (width 0.8) (layer "F.Cu") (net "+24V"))
 (segment (start 165.8 99.421382) (end 165.621382 99.6) (width 0.25) (layer "F.Cu") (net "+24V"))
 (segment (start 166.857236 96.6) (end 168 96.6) (width 0.25) (layer "F.Cu") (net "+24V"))
 (segment (start 175.25 86.75) (end 171.9625 86.75) (width 2) (layer "F.Cu") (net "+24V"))
 (segment (start 177 84.7075) (end 177 87.8) (width 2) (layer "F.Cu") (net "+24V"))
 (segment (start 170 86.7125) (end 170 84.46) (width 0.8) (layer "F.Cu") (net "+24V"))
 (segment (start 165 99.6) (end 164.8 99.4) (width 0.25) (layer "F.Cu") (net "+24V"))
 (segment (start 170.8 94) (end 168.65 94) (width 2) (layer "F.Cu") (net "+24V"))
 (segment (start 164.8 99.4) (end 164.8 98.45) (width 0.25) (layer "F.Cu") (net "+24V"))
 (segment (start 177 84.7075) (end 177 85) (width 2) (layer "F.Cu") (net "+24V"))
 (segment (start 168 96.6) (end 168.65 95.95) (width 0.25) (layer "F.Cu") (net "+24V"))
 (segment (start 170.95 86.7) (end 170.95 84.46) (width 0.8) (layer "F.Cu") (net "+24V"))
 (segment (start 171.5 87.2125) (end 171.4625 87.2125) (width 0.8) (layer "F.Cu") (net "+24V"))
 (segment (start 165.3 97.5) (end 164.4 96.6) (width 0.25) (layer "F.Cu") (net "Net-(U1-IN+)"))
 (segment (start 165.3 98.45) (end 165.3 97.5) (width 0.25) (layer "F.Cu") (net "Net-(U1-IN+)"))
 (segment (start 159.355 93.9225) (end 161.8275 93.9225) (width 2) (layer "F.Cu") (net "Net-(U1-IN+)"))
 (segment (start 161.905 94) (end 162.55 94) (width 2) (layer "F.Cu") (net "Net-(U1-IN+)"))
 (segment (start 161.8275 93.9225) (end 161.905 94) (width 2) (layer "F.Cu") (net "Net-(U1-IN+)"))
 (segment (start 164.4 96.6) (end 163.2 96.6) (width 0.25) (layer "F.Cu") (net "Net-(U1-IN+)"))
 (segment (start 162.6 96) (end 162.6 94.05) (width 0.25) (layer "F.Cu") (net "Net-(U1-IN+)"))
 (segment (start 163.2 96.6) (end 162.6 96) (width 0.25) (layer "F.Cu") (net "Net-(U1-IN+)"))
 (segment (start 162.6 94.05) (end 162.55 94) (width 0.25) (layer "F.Cu") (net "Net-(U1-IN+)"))
 (segment (start 162.55 94.35) (end 162.55 94) (width 0.25) (layer "F.Cu") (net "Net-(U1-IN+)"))
 (segment (start 182 94) (end 183.08 95.08) (width 0.45) (layer "F.Cu") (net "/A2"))
 (segment (start 174.2 99) (end 174.2 94.6) (width 0.45) (layer "F.Cu") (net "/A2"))
 (segment (start 161.3625 98.3625) (end 164.4125 101.4125) (width 0.45) (layer "F.Cu") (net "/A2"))
 (segment (start 174.2 94.6) (end 174.8 94) (width 0.45) (layer "F.Cu") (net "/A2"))
 (segment (start 171.7875 101.4125) (end 174.2 99) (width 0.45) (layer "F.Cu") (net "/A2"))
 (segment (start 159.6 98.3625) (end 161.3625 98.3625) (width 0.45) (layer "F.Cu") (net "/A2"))
 (segment (start 183.08 95.08) (end 183.08 95.925) (width 0.45) (layer "F.Cu") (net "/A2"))
 (segment (start 159.5625 98.4) (end 159.6 98.3625) (width 0.45) (layer "F.Cu") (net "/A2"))
 (segment (start 155.6 98.4) (end 157.6 98.4) (width 0.45) (layer "F.Cu") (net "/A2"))
 (segment (start 164.4125 101.4125) (end 171.7875 101.4125) (width 0.45) (layer "F.Cu") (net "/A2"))
 (segment (start 157.6 98.4) (end 159.5625 98.4) (width 0.45) (layer "F.Cu") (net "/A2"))
 (segment (start 174.8 94) (end 182 94) (width 0.45) (layer "F.Cu") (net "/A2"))
 (segment (start 167.8 104.4) (end 168.45 104.4) (width 0.45) (layer "F.Cu") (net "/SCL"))
 (segment (start 166.8 105.4) (end 167.8 104.4) (width 0.45) (layer "F.Cu") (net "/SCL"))
 (segment (start 171 104.4) (end 175.46 99.94) (width 0.45) (layer "F.Cu") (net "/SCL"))
 (segment (start 166.8 103.4) (end 167.8 104.4) (width 0.25) (layer "F.Cu") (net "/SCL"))
 (segment (start 166.8 102.75) (end 166.8 103.4) (width 0.25) (layer "F.Cu") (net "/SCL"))
 (segment (start 175.46 99.94) (end 175.46 96.76) (width 0.45) (layer "F.Cu") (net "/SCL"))
 (segment (start 166.8 106) (end 166.8 105.4) (width 0.45) (layer "F.Cu") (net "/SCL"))
 (segment (start 168.45 104.4) (end 171 104.4) (width 0.45) (layer "F.Cu") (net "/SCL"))
 (segment (start 150.4 98.4) (end 153.6 98.4) (width 0.45) (layer "F.Cu") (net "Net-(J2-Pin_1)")))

